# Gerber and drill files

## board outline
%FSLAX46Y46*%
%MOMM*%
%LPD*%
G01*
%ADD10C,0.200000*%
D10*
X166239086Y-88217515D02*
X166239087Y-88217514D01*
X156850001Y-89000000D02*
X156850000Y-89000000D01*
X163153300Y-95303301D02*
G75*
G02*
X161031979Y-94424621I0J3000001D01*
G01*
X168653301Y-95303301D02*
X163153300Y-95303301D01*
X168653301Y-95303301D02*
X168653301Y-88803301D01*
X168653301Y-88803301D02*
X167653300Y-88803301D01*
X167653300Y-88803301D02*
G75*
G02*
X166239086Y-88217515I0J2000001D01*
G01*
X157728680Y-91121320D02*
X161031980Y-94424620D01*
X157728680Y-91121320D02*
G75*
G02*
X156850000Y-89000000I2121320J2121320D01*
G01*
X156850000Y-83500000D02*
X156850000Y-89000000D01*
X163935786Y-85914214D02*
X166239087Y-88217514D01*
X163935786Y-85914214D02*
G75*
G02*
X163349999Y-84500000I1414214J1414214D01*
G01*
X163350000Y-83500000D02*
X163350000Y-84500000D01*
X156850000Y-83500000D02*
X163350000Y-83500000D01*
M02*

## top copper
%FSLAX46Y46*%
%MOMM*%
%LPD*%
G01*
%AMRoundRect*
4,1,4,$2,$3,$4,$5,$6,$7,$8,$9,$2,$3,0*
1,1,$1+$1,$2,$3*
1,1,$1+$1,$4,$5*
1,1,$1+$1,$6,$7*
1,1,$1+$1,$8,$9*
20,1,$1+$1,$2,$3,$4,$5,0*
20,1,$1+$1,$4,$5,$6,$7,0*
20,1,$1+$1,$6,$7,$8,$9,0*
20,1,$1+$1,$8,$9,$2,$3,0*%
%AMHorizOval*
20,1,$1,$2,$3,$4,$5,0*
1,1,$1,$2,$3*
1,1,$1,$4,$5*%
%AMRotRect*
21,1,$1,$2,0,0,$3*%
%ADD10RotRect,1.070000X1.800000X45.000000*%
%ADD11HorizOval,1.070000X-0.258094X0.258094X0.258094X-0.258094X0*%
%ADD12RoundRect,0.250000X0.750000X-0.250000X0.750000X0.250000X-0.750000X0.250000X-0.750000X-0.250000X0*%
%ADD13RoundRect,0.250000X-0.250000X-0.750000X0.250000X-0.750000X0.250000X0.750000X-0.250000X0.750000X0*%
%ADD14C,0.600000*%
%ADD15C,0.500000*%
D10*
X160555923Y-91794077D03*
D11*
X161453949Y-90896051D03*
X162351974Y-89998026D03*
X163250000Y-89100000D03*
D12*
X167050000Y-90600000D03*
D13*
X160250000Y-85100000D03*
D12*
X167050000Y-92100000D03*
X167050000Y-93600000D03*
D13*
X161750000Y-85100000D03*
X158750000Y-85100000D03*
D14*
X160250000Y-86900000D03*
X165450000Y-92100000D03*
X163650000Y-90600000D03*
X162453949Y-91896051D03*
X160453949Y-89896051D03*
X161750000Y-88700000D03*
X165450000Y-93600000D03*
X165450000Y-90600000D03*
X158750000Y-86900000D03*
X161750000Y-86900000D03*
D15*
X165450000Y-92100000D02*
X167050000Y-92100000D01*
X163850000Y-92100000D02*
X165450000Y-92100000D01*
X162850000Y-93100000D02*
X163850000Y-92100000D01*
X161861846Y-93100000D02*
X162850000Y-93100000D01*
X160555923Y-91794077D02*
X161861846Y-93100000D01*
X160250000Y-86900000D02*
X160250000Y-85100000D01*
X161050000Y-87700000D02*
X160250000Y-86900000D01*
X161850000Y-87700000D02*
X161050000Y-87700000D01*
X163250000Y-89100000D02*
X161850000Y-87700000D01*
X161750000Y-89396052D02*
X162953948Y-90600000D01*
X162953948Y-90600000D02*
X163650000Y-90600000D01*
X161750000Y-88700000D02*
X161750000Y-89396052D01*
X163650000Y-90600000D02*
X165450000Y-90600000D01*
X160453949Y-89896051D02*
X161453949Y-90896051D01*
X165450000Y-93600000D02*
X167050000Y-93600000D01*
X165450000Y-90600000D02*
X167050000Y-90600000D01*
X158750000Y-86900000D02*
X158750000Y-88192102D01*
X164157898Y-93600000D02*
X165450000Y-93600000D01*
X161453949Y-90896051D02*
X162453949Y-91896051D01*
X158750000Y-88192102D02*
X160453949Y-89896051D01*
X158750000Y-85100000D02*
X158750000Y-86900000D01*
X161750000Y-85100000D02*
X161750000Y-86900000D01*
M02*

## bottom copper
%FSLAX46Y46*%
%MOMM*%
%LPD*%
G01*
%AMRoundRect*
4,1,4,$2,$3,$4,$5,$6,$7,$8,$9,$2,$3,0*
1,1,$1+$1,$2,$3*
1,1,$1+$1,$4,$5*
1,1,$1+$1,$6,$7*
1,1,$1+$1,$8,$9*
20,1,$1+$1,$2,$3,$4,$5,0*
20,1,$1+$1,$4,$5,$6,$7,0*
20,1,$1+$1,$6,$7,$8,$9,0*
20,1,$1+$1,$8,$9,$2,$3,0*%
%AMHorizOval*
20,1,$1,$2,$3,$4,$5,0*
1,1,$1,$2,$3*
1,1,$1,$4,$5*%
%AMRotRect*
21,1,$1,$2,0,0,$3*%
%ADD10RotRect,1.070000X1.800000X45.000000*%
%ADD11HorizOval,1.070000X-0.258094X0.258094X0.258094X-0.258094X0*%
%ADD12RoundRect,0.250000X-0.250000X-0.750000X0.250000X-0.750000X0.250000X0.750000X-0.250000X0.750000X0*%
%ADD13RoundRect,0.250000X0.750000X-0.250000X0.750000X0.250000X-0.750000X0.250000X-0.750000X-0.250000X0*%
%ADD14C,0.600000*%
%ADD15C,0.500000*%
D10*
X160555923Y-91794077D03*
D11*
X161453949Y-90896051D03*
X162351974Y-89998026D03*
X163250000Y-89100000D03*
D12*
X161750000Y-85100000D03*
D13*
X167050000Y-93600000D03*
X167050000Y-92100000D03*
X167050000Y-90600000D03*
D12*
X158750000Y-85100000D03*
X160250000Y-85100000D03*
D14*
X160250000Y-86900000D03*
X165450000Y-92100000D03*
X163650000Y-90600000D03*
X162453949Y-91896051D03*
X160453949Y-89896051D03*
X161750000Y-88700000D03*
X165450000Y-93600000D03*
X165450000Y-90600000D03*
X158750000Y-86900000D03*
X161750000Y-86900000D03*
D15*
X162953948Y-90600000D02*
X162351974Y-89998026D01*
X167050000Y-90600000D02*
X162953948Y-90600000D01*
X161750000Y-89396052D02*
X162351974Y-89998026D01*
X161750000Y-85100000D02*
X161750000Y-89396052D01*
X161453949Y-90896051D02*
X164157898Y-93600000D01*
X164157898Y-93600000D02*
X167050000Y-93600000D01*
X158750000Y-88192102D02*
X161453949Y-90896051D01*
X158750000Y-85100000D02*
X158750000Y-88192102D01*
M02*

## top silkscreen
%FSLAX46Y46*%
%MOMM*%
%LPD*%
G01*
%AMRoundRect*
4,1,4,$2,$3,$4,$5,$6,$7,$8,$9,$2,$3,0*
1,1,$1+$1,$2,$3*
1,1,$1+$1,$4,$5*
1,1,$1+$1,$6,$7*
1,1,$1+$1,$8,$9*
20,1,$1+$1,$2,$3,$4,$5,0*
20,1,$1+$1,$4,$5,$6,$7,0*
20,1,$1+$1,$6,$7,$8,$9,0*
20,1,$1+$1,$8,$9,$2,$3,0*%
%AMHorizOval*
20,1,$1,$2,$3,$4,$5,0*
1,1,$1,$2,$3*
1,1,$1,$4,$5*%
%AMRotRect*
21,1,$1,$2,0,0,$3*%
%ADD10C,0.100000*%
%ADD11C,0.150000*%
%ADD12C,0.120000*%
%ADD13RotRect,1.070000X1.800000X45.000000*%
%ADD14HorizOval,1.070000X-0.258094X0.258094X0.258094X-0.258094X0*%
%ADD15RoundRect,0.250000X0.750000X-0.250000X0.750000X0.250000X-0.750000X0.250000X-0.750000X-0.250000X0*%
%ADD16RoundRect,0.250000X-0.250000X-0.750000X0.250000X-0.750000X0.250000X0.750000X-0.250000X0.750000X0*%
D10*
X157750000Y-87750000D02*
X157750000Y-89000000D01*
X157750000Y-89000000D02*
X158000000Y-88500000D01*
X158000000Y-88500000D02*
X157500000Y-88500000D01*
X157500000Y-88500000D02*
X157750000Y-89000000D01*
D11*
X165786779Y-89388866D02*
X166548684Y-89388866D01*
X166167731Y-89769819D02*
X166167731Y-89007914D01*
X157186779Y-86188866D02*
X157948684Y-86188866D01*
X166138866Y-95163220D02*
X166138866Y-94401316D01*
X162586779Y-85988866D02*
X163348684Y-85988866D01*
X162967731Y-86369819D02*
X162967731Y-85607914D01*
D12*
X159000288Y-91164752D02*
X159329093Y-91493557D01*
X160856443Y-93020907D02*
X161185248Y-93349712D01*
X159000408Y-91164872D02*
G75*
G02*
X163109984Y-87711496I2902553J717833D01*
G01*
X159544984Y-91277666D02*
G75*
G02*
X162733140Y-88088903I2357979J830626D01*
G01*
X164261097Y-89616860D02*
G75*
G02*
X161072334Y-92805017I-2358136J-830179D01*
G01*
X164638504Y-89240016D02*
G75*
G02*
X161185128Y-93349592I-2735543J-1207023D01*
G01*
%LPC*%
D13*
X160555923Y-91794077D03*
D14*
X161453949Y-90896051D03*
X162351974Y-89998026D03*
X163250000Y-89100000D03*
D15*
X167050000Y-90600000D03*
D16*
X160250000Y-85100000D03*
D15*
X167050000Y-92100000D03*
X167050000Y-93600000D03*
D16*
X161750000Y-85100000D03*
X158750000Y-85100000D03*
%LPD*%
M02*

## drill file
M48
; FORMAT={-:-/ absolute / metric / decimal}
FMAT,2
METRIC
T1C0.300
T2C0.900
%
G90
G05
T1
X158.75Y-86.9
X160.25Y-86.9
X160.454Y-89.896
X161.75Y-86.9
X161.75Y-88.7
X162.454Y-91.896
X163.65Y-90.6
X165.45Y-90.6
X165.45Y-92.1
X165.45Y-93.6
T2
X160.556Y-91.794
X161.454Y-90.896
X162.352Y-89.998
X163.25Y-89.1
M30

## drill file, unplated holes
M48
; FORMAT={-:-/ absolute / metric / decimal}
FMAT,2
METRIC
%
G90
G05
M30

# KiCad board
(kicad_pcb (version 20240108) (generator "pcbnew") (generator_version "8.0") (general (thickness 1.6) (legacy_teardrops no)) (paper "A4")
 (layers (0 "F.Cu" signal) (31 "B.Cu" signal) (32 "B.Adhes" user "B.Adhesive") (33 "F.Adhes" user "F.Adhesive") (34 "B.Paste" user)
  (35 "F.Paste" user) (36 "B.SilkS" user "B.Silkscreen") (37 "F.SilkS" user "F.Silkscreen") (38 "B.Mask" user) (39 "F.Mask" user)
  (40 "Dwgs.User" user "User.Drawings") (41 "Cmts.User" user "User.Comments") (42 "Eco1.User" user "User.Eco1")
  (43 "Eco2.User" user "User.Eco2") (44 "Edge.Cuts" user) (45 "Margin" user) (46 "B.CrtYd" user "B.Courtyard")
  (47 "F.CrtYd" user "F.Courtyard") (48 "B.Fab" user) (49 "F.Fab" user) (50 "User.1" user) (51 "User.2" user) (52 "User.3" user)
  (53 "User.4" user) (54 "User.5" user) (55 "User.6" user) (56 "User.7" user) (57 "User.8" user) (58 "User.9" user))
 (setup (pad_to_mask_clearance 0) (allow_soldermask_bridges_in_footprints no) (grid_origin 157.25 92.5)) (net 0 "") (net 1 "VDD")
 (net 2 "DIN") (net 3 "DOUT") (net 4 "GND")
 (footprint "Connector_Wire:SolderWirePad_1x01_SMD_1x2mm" (layer "F.Cu") (at 167.05 90.6 90)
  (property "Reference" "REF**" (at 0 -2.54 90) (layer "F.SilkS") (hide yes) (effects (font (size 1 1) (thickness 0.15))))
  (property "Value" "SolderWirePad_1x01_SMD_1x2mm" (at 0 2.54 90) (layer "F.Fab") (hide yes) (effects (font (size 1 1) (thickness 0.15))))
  (pad "1" smd roundrect (at 0 0 90) (size 1 2) (layers "F.Cu" "F.Paste" "F.Mask") (roundrect_rratio 0.25) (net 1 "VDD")))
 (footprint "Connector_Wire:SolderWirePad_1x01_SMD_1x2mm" (layer "F.Cu") (at 160.25 85.1)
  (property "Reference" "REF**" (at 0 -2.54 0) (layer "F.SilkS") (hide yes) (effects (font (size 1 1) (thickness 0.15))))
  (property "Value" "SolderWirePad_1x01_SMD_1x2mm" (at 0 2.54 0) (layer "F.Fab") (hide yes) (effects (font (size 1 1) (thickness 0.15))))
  (pad "1" smd roundrect (at 0 0) (size 1 2) (layers "F.Cu" "F.Paste" "F.Mask") (roundrect_rratio 0.25) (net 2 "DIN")))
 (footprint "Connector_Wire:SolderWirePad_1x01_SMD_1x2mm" (layer "F.Cu") (at 167.05 92.1 90)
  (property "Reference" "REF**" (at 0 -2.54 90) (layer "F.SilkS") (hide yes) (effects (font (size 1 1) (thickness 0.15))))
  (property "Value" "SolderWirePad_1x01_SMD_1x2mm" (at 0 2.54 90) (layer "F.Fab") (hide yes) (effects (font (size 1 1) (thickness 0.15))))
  (pad "1" smd roundrect (at 0 0 90) (size 1 2) (layers "F.Cu" "F.Paste" "F.Mask") (roundrect_rratio 0.25) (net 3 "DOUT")))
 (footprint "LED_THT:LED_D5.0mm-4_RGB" (layer "F.Cu") (at 160.555923 91.794077 45)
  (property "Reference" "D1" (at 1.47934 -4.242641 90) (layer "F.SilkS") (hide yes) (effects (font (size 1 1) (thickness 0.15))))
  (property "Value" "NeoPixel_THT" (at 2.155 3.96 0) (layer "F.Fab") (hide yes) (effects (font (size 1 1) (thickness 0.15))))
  (fp_line (start -0.655 -1.545) (end -0.655 -1.08) (stroke (width 0.12) (type solid)) (layer "F.SilkS"))
  (fp_line (start -0.655 1.08) (end -0.655 1.545) (stroke (width 0.12) (type solid)) (layer "F.SilkS"))
  (fp_arc (start -0.655 -1.54483) (mid 2.163456 -2.978808) (end 4.692815 -1.080827) (stroke (width 0.12) (type solid)) (layer "F.SilkS"))
  (fp_arc (start -0.349684 -1.08) (mid 1.904762 -2.499999) (end 4.159479 -1.080429) (stroke (width 0.12) (type solid)) (layer "F.SilkS"))
  (fp_arc (start 4.159479 1.080429) (mid 1.904762 2.5) (end -0.349684 1.08) (stroke (width 0.12) (type solid)) (layer "F.SilkS"))
  (fp_arc (start 4.692815 1.080827) (mid 2.163456 2.978808) (end -0.655 1.54483) (stroke (width 0.12) (type solid)) (layer "F.SilkS"))
  (pad "1" thru_hole rect (at 0 0 45) (size 1.07 1.8) (drill 0.9) (layers "*.Cu" "*.Mask") (remove_unused_layers no) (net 3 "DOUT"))
  (pad "2" thru_hole oval (at 1.270001 0 45) (size 1.07 1.8) (drill 0.9) (layers "*.Cu" "*.Mask") (remove_unused_layers no) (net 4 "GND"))
  (pad "3" thru_hole oval (at 2.54 0 45) (size 1.07 1.8) (drill 0.9) (layers "*.Cu" "*.Mask") (remove_unused_layers no) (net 1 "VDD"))
  (pad "4" thru_hole oval (at 3.81 0 45) (size 1.07 1.8) (drill 0.9) (layers "*.Cu" "*.Mask") (remove_unused_layers no) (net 2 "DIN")))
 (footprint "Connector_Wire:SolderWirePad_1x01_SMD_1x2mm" (layer "F.Cu") (at 167.05 93.6 90)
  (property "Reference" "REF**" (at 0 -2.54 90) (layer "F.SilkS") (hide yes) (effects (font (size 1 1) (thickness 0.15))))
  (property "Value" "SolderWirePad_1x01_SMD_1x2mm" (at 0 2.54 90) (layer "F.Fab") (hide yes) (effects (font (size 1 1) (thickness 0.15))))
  (pad "1" smd roundrect (at 0 0 90) (size 1 2) (layers "F.Cu" "F.Paste" "F.Mask") (roundrect_rratio 0.25) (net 4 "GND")))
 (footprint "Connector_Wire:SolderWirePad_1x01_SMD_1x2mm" (layer "F.Cu") (at 161.75 85.1)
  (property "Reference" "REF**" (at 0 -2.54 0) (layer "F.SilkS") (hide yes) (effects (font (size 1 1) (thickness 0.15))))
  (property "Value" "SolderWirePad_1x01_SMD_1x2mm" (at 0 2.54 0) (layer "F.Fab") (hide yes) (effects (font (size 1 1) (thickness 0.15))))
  (pad "1" smd roundrect (at 0 0) (size 1 2) (layers "F.Cu" "F.Paste" "F.Mask") (roundrect_rratio 0.25) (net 1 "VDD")))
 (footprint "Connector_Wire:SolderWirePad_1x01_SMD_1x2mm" (layer "F.Cu") (at 158.75 85.1)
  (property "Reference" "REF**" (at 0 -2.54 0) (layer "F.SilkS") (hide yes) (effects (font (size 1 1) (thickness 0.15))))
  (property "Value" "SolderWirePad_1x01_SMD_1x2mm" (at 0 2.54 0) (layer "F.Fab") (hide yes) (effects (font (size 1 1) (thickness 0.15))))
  (pad "1" smd roundrect (at 0 0) (size 1 2) (layers "F.Cu" "F.Paste" "F.Mask") (roundrect_rratio 0.25) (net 4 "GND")))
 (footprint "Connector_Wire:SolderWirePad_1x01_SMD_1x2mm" (layer "B.Cu") (at 161.75 85.1)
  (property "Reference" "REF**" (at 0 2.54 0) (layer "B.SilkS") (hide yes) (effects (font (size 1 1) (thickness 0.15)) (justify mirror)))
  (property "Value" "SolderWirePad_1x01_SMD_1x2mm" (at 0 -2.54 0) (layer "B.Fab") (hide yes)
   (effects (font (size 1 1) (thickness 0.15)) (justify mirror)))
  (pad "1" smd roundrect (at 0 0) (size 1 2) (layers "B.Cu" "B.Paste" "B.Mask") (roundrect_rratio 0.25) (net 1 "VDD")))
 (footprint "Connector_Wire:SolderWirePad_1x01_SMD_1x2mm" (layer "B.Cu") (at 167.05 93.6 90)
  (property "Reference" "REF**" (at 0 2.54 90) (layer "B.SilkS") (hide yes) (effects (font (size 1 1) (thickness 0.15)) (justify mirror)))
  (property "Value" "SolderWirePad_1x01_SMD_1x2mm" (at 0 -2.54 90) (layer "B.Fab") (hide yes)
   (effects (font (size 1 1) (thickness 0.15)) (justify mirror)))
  (pad "1" smd roundrect (at 0 0 90) (size 1 2) (layers "B.Cu" "B.Paste" "B.Mask") (roundrect_rratio 0.25) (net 4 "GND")))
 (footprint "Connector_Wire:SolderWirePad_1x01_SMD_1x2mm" (layer "B.Cu") (at 167.05 92.1 90)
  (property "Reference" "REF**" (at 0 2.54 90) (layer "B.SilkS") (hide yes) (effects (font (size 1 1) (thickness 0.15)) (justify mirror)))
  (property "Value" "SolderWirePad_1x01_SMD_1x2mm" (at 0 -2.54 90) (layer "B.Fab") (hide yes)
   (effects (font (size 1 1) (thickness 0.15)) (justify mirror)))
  (pad "1" smd roundrect (at 0 0 90) (size 1 2) (layers "B.Cu" "B.Paste" "B.Mask") (roundrect_rratio 0.25) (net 3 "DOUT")))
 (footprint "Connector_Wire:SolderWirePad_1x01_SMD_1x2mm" (layer "B.Cu") (at 167.05 90.6 90)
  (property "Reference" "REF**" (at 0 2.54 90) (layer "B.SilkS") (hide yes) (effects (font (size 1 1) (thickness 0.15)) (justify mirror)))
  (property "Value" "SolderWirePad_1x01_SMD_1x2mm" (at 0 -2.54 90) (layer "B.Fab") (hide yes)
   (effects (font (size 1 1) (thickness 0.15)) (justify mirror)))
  (pad "1" smd roundrect (at 0 0 90) (size 1 2) (layers "B.Cu" "B.Paste" "B.Mask") (roundrect_rratio 0.25) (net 1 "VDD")))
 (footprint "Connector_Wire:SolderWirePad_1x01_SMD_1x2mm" (layer "B.Cu") (at 158.75 85.1)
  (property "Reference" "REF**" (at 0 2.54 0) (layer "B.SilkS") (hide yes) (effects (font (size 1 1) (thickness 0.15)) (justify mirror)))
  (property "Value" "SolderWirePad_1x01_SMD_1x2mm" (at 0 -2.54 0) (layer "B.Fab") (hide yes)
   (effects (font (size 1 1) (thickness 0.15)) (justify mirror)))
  (pad "1" smd roundrect (at 0 0) (size 1 2) (layers "B.Cu" "B.Paste" "B.Mask") (roundrect_rratio 0.25) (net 4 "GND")))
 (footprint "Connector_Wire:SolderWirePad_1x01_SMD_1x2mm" (layer "B.Cu") (at 160.25 85.1)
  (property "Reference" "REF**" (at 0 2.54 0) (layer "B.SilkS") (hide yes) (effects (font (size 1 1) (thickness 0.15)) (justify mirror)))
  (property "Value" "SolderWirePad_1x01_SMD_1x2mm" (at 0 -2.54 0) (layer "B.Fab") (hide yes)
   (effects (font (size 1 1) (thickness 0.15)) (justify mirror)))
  (pad "1" smd roundrect (at 0 0) (size 1 2) (layers "B.Cu" "B.Paste" "B.Mask") (roundrect_rratio 0.25) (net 2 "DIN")))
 (gr_line (start 157.75 87.75) (end 157.75 89) (stroke (width 0.1) (type default)) (layer "F.SilkS"))
 (gr_line (start 157.75 89) (end 158 88.5) (stroke (width 0.1) (type default)) (layer "F.SilkS"))
 (gr_line (start 158 88.5) (end 157.5 88.5) (stroke (width 0.1) (type default)) (layer "F.SilkS"))
 (gr_line (start 157.5 88.5) (end 157.75 89) (stroke (width 0.1) (type default)) (layer "F.SilkS"))
 (gr_arc (start 157.72868 91.12132) (mid 157.078362 90.14805) (end 156.850001 89) (stroke (width 0.2) (type default)) (layer "Edge.Cuts"))
 (gr_line (start 168.653301 95.303301) (end 168.653301 88.803301) (stroke (width 0.2) (type default)) (layer "Edge.Cuts"))
 (gr_line (start 156.85 83.5) (end 163.35 83.5) (stroke (width 0.2) (type default)) (layer "Edge.Cuts"))
 (gr_line (start 156.850001 89) (end 156.85 89) (stroke (width 0.2) (type default)) (layer "Edge.Cuts"))
 (gr_line (start 168.653301 88.803301) (end 167.6533 88.803301) (stroke (width 0.2) (type default)) (layer "Edge.Cuts"))
 (gr_arc (start 163.1533 95.303301) (mid 162.005249 95.07494) (end 161.03198 94.42462) (stroke (width 0.2) (type default))
  (layer "Edge.Cuts"))
 (gr_arc (start 167.6533 88.803301) (mid 166.887933 88.65106) (end 166.239086 88.217515) (stroke (width 0.2) (type default))
  (layer "Edge.Cuts"))
 (gr_line (start 163.35 83.5) (end 163.35 84.5) (stroke (width 0.2) (type default)) (layer "Edge.Cuts"))
 (gr_arc (start 163.935786 85.914214) (mid 163.50224 85.265367) (end 163.35 84.5) (stroke (width 0.2) (type default)) (layer "Edge.Cuts"))
 (gr_line (start 168.653301 95.303301) (end 163.1533 95.303301) (stroke (width 0.2) (type default)) (layer "Edge.Cuts"))
 (gr_line (start 156.85 83.5) (end 156.85 89) (stroke (width 0.2) (type default)) (layer "Edge.Cuts"))
 (gr_line (start 166.239086 88.217515) (end 166.239087 88.217514) (stroke (width 0.2) (type default)) (layer "Edge.Cuts"))
 (gr_line (start 157.72868 91.12132) (end 161.03198 94.42462) (stroke (width 0.2) (type default)) (layer "Edge.Cuts"))
 (gr_line (start 163.935786 85.914214) (end 166.239087 88.217514) (stroke (width 0.2) (type default)) (layer "Edge.Cuts"))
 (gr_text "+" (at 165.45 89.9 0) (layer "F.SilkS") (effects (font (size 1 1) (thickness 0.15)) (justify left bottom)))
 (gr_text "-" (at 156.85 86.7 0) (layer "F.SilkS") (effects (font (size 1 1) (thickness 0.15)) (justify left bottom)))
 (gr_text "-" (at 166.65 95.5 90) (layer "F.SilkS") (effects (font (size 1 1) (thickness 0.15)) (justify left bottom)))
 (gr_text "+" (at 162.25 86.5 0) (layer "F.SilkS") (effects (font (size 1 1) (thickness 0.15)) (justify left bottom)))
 (segment (start 165.45 93.6) (end 167.05 93.6) (width 0.5) (layer "F.Cu") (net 4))
 (segment (start 164.157898 93.6) (end 165.45 93.6) (width 0.5) (layer "F.Cu") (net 4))
 (segment (start 160.453949 89.896051) (end 161.453949 90.896051) (width 0.5) (layer "F.Cu") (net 4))
 (segment (start 158.75 86.9) (end 158.75 88.192102) (width 0.5) (layer "F.Cu") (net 4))
 (segment (start 158.75 88.192102) (end 160.453949 89.896051) (width 0.5) (layer "F.Cu") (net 4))
 (segment (start 161.453949 90.896051) (end 162.453949 91.896051) (width 0.5) (layer "F.Cu") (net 4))
 (segment (start 158.75 85.1) (end 158.75 86.9) (width 0.5) (layer "F.Cu") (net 4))
 (via (at 160.453949 89.896051) (size 0.6) (drill 0.3) (layers "F.Cu" "B.Cu") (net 4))
 (via (at 165.45 93.6) (size 0.6) (drill 0.3) (layers "F.Cu" "B.Cu") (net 4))
 (via (at 162.453949 91.896051) (size 0.6) (drill 0.3) (layers "F.Cu" "B.Cu") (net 4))
 (via (at 158.75 86.9) (size 0.6) (drill 0.3) (layers "F.Cu" "B.Cu") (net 4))
 (segment (start 164.157898 93.6) (end 167.05 93.6) (width 0.5) (layer "B.Cu") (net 4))
 (segment (start 158.75 85.1) (end 158.75 88.192102) (width 0.5) (layer "B.Cu") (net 4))
 (segment (start 161.453949 90.896051) (end 164.157898 93.6) (width 0.5) (layer "B.Cu") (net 4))
 (segment (start 158.75 88.192102) (end 161.453949 90.896051) (width 0.5) (layer "B.Cu") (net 4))
 (segment (start 163.25 89.1) (end 161.85 87.7) (width 0.5) (layer "F.Cu") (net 2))
 (segment (start 160.25 86.9) (end 160.25 85.1) (width 0.5) (layer "F.Cu") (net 2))
 (segment (start 161.85 87.7) (end 161.05 87.7) (width 0.5) (layer "F.Cu") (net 2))
 (segment (start 161.05 87.7) (end 160.25 86.9) (width 0.5) (layer "F.Cu") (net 2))
 (via (at 160.25 86.9) (size 0.6) (drill 0.3) (layers "F.Cu" "B.Cu") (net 2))
 (segment (start 161.861846 93.1) (end 162.85 93.1) (width 0.5) (layer "F.Cu") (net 3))
 (segment (start 163.85 92.1) (end 165.45 92.1) (width 0.5) (layer "F.Cu") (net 3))
 (segment (start 160.555923 91.794077) (end 161.861846 93.1) (width 0.5) (layer "F.Cu") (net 3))
 (segment (start 165.45 92.1) (end 167.05 92.1) (width 0.5) (layer "F.Cu") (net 3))
 (segment (start 162.85 93.1) (end 163.85 92.1) (width 0.5) (layer "F.Cu") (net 3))
 (via (at 165.45 92.1) (size 0.6) (drill 0.3) (layers "F.Cu" "B.Cu") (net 3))
 (segment (start 161.75 89.396052) (end 162.953948 90.6) (width 0.5) (layer "F.Cu") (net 1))
 (segment (start 163.65 90.6) (end 165.45 90.6) (width 0.5) (layer "F.Cu") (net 1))
 (segment (start 165.45 90.6) (end 167.05 90.6) (width 0.5) (layer "F.Cu") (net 1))
 (segment (start 162.953948 90.6) (end 163.65 90.6) (width 0.5) (layer "F.Cu") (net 1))
 (segment (start 161.75 85.1) (end 161.75 86.9) (width 0.5) (layer "F.Cu") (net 1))
 (segment (start 161.75 88.7) (end 161.75 89.396052) (width 0.5) (layer "F.Cu") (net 1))
 (via (at 161.75 86.9) (size 0.6) (drill 0.3) (layers "F.Cu" "B.Cu") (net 1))
 (via (at 163.65 90.6) (size 0.6) (drill 0.3) (layers "F.Cu" "B.Cu") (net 1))
 (via (at 161.75 88.7) (size 0.6) (drill 0.3) (layers "F.Cu" "B.Cu") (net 1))
 (via (at 165.45 90.6) (size 0.6) (drill 0.3) (layers "F.Cu" "B.Cu") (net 1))
 (segment (start 162.953948 90.6) (end 162.351974 89.998026) (width 0.5) (layer "B.Cu") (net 1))
 (segment (start 161.75 85.1) (end 161.75 89.396052) (width 0.5) (layer "B.Cu") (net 1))
 (segment (start 161.75 89.396052) (end 162.351974 89.998026) (width 0.5) (layer "B.Cu") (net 1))
 (segment (start 167.05 90.6) (end 162.953948 90.6) (width 0.5) (layer "B.Cu") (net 1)))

